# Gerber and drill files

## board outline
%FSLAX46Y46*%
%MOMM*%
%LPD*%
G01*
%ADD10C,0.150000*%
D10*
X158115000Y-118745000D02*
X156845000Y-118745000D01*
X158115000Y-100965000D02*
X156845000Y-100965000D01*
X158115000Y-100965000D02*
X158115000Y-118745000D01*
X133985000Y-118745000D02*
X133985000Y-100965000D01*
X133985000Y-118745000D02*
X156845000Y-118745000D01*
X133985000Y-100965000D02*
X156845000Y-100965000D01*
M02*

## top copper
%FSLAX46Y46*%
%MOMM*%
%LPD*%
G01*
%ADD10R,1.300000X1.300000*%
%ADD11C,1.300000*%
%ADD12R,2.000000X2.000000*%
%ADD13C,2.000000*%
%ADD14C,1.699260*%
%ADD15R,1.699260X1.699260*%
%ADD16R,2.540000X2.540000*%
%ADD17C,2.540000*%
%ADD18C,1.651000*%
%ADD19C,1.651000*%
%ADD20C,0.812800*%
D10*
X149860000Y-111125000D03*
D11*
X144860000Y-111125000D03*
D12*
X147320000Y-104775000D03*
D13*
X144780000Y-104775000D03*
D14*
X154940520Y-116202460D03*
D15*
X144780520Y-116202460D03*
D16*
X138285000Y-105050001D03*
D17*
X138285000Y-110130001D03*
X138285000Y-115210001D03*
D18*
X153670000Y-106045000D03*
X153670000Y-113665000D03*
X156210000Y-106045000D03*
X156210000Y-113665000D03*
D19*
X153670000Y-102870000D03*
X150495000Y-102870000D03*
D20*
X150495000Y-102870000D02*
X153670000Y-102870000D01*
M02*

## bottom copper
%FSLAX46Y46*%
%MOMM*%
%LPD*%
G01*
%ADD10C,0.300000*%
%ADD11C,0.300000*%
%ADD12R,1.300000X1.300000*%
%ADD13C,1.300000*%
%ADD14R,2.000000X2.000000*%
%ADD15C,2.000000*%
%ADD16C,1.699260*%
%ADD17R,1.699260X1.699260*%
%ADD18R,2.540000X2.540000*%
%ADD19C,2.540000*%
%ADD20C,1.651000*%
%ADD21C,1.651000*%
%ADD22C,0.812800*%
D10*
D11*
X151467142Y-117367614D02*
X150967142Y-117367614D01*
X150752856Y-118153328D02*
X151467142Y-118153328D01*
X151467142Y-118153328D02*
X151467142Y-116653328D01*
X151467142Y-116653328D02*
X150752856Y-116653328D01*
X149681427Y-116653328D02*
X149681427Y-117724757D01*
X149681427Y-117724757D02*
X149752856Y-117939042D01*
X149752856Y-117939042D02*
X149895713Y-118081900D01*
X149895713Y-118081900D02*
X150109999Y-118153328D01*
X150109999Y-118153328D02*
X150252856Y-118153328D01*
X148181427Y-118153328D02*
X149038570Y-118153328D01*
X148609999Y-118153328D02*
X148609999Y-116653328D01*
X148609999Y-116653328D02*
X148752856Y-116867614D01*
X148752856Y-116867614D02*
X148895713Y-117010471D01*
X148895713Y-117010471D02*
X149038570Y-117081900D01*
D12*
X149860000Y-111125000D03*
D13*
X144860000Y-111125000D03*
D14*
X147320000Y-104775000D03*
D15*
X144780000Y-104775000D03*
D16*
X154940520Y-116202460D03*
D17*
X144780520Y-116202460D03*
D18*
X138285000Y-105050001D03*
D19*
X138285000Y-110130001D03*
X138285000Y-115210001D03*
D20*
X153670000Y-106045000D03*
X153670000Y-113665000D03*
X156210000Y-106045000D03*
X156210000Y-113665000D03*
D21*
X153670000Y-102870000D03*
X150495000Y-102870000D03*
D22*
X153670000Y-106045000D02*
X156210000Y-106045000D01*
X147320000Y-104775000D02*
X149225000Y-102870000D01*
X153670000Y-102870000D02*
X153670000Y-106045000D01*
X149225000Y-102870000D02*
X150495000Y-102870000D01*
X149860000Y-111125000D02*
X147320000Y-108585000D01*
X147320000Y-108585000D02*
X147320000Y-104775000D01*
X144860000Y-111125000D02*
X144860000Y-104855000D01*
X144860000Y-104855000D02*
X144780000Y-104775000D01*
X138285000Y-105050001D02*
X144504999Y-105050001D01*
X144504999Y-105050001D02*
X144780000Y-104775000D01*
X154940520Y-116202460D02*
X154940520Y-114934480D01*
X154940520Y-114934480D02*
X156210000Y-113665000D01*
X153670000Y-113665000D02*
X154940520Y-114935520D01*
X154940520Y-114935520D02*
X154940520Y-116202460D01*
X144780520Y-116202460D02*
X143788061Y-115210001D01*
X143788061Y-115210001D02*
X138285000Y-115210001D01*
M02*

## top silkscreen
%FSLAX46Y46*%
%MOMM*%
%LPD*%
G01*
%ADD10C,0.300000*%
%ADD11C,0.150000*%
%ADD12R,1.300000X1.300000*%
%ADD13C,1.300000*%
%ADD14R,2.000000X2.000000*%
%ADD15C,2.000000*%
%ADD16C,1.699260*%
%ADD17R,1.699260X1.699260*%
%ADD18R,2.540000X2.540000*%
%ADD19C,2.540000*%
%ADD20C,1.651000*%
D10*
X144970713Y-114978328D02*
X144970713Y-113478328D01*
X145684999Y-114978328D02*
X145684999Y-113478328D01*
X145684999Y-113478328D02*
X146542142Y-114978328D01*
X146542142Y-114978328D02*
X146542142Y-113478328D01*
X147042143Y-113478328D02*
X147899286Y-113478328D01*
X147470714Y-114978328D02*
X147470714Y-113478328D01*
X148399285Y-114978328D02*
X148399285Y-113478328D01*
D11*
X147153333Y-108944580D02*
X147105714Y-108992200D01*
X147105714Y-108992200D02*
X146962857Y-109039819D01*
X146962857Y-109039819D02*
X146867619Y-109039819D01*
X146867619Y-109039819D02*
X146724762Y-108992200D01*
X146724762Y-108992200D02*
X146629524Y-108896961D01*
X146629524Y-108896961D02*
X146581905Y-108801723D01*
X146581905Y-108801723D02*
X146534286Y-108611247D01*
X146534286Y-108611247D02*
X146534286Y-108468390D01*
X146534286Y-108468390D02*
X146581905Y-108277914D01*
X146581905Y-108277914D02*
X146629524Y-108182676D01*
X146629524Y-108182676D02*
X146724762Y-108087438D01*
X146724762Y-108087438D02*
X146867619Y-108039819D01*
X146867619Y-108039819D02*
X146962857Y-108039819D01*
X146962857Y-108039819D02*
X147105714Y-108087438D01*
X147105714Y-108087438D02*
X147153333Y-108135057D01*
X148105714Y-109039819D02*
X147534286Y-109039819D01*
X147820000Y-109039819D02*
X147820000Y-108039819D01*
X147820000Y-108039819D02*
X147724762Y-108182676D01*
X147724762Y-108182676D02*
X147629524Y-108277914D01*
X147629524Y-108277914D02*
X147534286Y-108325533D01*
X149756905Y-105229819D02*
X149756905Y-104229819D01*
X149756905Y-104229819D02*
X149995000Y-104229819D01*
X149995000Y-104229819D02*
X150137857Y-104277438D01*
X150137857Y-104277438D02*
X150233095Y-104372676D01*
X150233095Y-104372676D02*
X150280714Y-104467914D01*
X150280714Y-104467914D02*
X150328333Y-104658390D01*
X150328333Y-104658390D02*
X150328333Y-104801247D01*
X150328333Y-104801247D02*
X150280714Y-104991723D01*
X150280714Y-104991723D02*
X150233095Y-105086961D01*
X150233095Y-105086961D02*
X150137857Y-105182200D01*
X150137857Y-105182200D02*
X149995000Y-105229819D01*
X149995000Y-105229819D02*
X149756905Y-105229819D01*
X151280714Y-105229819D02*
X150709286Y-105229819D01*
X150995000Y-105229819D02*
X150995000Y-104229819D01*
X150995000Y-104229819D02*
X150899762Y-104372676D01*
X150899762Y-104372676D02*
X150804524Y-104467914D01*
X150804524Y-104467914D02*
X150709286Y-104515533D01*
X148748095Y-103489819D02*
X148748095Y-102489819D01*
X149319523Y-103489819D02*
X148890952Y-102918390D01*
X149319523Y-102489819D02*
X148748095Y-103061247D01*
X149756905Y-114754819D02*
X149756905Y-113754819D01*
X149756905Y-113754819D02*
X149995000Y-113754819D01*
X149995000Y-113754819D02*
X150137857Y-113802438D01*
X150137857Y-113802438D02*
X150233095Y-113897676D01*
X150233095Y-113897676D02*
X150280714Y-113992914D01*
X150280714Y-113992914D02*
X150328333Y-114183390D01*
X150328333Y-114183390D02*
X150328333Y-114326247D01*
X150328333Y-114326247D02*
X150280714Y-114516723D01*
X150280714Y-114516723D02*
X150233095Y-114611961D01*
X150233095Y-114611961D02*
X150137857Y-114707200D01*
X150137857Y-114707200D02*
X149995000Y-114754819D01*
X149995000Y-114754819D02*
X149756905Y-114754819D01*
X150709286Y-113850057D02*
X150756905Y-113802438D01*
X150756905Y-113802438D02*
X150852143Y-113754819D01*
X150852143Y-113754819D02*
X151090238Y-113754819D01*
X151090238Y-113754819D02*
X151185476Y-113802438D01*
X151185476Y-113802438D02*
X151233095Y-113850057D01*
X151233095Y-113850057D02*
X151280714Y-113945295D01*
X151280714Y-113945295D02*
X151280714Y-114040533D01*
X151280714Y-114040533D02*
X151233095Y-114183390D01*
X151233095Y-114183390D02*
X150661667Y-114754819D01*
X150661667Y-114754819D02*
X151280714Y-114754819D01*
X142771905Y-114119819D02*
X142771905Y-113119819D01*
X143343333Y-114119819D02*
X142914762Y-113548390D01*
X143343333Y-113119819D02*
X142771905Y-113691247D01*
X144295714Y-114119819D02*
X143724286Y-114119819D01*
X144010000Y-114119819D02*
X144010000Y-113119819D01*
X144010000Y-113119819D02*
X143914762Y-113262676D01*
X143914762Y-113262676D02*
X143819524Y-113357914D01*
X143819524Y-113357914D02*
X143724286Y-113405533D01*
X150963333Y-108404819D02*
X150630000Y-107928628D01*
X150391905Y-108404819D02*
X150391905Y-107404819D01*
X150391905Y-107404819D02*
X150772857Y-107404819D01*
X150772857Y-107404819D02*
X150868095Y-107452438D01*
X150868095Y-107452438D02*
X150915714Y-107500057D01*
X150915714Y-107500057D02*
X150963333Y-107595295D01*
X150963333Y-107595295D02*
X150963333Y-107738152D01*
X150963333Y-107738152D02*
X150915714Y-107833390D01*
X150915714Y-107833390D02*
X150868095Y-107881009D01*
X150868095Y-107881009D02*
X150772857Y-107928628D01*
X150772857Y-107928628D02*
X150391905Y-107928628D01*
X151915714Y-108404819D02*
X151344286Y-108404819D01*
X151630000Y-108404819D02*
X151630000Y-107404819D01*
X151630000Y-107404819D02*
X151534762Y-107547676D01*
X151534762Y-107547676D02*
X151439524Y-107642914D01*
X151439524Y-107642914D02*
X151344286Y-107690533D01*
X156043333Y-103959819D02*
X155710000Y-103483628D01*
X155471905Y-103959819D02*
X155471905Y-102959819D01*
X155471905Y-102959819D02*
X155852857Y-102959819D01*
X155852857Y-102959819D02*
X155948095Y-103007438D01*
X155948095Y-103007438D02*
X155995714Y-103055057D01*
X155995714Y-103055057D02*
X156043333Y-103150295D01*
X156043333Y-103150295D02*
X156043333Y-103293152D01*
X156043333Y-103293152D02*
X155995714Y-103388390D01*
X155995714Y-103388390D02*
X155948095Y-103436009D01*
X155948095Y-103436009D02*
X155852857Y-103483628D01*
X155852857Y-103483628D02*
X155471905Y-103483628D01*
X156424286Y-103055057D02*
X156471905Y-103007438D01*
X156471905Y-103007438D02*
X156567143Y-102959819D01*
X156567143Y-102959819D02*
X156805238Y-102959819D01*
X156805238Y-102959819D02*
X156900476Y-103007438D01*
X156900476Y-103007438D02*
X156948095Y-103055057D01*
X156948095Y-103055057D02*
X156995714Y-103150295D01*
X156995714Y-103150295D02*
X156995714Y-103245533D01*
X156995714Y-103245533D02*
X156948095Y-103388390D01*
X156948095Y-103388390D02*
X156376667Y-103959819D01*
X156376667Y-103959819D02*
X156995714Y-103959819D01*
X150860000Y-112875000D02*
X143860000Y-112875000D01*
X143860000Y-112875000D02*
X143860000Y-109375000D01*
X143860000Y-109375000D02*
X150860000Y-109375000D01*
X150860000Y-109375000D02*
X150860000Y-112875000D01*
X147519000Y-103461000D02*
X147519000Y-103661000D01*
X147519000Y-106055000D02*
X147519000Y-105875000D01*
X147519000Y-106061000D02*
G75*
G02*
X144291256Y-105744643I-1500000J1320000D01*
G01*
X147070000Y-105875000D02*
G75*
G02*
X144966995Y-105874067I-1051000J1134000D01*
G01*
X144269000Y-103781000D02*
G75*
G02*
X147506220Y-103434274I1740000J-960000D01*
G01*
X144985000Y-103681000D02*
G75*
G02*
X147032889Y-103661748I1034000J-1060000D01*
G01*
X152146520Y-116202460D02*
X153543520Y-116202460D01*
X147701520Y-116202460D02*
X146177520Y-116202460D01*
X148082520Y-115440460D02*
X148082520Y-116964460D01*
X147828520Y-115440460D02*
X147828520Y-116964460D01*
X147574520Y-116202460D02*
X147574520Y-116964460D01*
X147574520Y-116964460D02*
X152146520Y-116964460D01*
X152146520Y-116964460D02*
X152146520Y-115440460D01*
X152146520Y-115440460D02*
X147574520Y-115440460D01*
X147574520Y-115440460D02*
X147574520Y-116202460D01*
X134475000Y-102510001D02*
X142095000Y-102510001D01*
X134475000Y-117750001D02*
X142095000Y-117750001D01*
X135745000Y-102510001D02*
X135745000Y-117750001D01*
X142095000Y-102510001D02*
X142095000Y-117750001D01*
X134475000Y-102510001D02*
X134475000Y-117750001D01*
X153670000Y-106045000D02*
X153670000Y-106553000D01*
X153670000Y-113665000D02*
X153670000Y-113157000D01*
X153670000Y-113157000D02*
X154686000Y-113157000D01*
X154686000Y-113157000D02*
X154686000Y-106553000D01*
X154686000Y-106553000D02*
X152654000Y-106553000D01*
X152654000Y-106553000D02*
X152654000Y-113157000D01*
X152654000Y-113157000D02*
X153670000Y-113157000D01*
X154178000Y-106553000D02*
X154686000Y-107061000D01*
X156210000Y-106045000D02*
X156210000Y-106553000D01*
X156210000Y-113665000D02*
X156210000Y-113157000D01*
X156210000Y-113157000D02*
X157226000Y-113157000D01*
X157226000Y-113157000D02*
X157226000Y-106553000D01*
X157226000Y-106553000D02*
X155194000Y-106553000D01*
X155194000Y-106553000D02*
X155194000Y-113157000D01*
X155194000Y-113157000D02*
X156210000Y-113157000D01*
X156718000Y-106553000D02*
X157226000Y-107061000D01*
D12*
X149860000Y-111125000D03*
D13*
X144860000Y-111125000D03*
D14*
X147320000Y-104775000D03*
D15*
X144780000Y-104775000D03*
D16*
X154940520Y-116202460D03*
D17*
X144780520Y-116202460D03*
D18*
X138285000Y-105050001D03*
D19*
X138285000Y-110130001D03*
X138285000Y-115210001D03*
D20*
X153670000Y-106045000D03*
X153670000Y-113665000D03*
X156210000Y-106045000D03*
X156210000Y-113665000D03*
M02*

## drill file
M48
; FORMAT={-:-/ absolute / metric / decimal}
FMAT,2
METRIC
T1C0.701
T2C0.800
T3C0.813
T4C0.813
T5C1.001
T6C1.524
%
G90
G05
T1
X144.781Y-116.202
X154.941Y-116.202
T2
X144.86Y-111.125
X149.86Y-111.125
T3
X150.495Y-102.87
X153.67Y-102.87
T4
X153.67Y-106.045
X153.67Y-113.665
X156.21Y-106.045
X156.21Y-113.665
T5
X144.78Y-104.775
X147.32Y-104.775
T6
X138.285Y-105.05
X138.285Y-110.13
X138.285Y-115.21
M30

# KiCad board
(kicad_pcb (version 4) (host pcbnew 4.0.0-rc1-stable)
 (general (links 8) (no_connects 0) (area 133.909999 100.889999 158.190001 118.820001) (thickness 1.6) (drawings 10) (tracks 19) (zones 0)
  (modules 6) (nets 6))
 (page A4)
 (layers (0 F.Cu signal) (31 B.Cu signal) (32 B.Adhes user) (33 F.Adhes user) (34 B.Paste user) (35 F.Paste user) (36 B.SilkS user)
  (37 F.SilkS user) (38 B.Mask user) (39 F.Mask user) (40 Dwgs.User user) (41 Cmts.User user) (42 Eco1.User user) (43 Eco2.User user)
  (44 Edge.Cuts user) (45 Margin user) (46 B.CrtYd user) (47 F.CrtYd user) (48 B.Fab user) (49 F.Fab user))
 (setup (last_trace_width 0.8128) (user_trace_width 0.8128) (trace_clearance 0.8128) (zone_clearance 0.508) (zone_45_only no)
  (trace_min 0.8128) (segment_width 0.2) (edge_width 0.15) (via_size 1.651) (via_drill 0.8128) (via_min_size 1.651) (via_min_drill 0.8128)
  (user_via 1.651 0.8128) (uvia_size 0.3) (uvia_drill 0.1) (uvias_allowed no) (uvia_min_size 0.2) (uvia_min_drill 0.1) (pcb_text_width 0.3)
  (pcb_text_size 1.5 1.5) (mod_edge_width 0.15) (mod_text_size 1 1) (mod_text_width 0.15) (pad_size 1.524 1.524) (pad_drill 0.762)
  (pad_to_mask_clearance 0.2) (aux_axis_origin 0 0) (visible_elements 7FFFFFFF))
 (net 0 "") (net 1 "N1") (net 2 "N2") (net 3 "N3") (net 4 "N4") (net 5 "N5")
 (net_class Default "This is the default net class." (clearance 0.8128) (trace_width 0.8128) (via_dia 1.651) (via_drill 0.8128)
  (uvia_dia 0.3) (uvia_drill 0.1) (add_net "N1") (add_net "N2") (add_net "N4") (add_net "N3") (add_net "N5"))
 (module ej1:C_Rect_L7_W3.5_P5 (layer F.Cu) (at 149.86 111.125 180)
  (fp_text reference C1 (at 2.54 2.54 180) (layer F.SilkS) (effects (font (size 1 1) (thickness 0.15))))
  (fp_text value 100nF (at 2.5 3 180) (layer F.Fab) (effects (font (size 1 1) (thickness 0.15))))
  (fp_line (start -1 -1.75) (end 6 -1.75) (layer F.SilkS) (width 0.15))
  (fp_line (start 6 -1.75) (end 6 1.75) (layer F.SilkS) (width 0.15))
  (fp_line (start 6 1.75) (end -1 1.75) (layer F.SilkS) (width 0.15))
  (fp_line (start -1 1.75) (end -1 -1.75) (layer F.SilkS) (width 0.15))
  (pad 1 thru_hole rect (at 0 0 180) (size 1.3 1.3) (drill 0.8) (layers *.Cu *.Mask F.SilkS) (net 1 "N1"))
  (pad 2 thru_hole circle (at 5 0 180) (size 1.3 1.3) (drill 0.8) (layers *.Cu *.Mask F.SilkS) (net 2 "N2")))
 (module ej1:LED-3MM (layer F.Cu) (at 147.32 104.775 180)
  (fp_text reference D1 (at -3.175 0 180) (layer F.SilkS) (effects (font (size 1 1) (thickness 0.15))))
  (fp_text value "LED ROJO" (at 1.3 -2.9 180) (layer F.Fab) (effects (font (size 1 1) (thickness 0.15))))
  (fp_line (start -0.199 1.314) (end -0.199 1.114) (layer F.SilkS) (width 0.15))
  (fp_line (start -0.199 -1.28) (end -0.199 -1.1) (layer F.SilkS) (width 0.15))
  (fp_arc (start 1.301 0.034) (end -0.199 -1.286) (angle 108.5) (layer F.SilkS) (width 0.15))
  (fp_arc (start 1.301 0.034) (end 0.25 -1.1) (angle 85.7) (layer F.SilkS) (width 0.15))
  (fp_arc (start 1.311 0.034) (end 3.051 0.994) (angle 110) (layer F.SilkS) (width 0.15))
  (fp_arc (start 1.301 0.034) (end 2.335 1.094) (angle 87.5) (layer F.SilkS) (width 0.15))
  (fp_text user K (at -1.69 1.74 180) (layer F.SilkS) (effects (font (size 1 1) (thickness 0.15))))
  (pad 1 thru_hole rect (at 0 0 270) (size 2 2) (drill 1.00076) (layers *.Cu *.Mask F.SilkS) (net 1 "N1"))
  (pad 2 thru_hole circle (at 2.54 0 180) (size 2 2) (drill 1.00076) (layers *.Cu *.Mask F.SilkS) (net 2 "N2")))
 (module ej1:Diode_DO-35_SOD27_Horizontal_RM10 (layer F.Cu) (at 144.78 116.205)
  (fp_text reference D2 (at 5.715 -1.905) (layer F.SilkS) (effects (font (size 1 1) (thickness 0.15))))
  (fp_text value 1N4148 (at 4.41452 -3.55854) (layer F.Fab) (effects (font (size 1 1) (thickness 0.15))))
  (fp_line (start 7.36652 -0.00254) (end 8.76352 -0.00254) (layer F.SilkS) (width 0.15))
  (fp_line (start 2.92152 -0.00254) (end 1.39752 -0.00254) (layer F.SilkS) (width 0.15))
  (fp_line (start 3.30252 -0.76454) (end 3.30252 0.75946) (layer F.SilkS) (width 0.15))
  (fp_line (start 3.04852 -0.76454) (end 3.04852 0.75946) (layer F.SilkS) (width 0.15))
  (fp_line (start 2.79452 -0.00254) (end 2.79452 0.75946) (layer F.SilkS) (width 0.15))
  (fp_line (start 2.79452 0.75946) (end 7.36652 0.75946) (layer F.SilkS) (width 0.15))
  (fp_line (start 7.36652 0.75946) (end 7.36652 -0.76454) (layer F.SilkS) (width 0.15))
  (fp_line (start 7.36652 -0.76454) (end 2.79452 -0.76454) (layer F.SilkS) (width 0.15))
  (fp_line (start 2.79452 -0.76454) (end 2.79452 -0.00254) (layer F.SilkS) (width 0.15))
  (pad 2 thru_hole circle (at 10.16052 -0.00254 180) (size 1.69926 1.69926) (drill 0.70104) (layers *.Cu *.Mask F.SilkS) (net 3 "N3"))
  (pad 1 thru_hole rect (at 0.00052 -0.00254 180) (size 1.69926 1.69926) (drill 0.70104) (layers *.Cu *.Mask F.SilkS) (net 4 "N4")))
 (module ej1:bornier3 (layer F.Cu) (at 138.285 110.130001 270)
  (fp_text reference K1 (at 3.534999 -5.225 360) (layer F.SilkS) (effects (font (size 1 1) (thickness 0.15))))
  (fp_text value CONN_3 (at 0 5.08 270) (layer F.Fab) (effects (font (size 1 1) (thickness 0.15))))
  (fp_line (start -7.62 3.81) (end -7.62 -3.81) (layer F.SilkS) (width 0.15))
  (fp_line (start 7.62 3.81) (end 7.62 -3.81) (layer F.SilkS) (width 0.15))
  (fp_line (start -7.62 2.54) (end 7.62 2.54) (layer F.SilkS) (width 0.15))
  (fp_line (start -7.62 -3.81) (end 7.62 -3.81) (layer F.SilkS) (width 0.15))
  (fp_line (start -7.62 3.81) (end 7.62 3.81) (layer F.SilkS) (width 0.15))
  (pad 1 thru_hole rect (at -5.08 0 270) (size 2.54 2.54) (drill 1.524) (layers *.Cu *.Mask F.SilkS) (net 2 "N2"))
  (pad 2 thru_hole circle (at 0 0 270) (size 2.54 2.54) (drill 1.524) (layers *.Cu *.Mask F.SilkS) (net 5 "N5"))
  (pad 3 thru_hole circle (at 5.08 0 270) (size 2.54 2.54) (drill 1.524) (layers *.Cu *.Mask F.SilkS) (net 4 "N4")))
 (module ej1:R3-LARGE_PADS (layer F.Cu) (at 153.67 109.855 270)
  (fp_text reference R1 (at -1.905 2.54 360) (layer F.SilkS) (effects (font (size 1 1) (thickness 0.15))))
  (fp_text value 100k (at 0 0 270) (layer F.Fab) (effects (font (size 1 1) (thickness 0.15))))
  (fp_line (start -3.81 0) (end -3.302 0) (layer F.SilkS) (width 0.15))
  (fp_line (start 3.81 0) (end 3.302 0) (layer F.SilkS) (width 0.15))
  (fp_line (start 3.302 0) (end 3.302 -1.016) (layer F.SilkS) (width 0.15))
  (fp_line (start 3.302 -1.016) (end -3.302 -1.016) (layer F.SilkS) (width 0.15))
  (fp_line (start -3.302 -1.016) (end -3.302 1.016) (layer F.SilkS) (width 0.15))
  (fp_line (start -3.302 1.016) (end 3.302 1.016) (layer F.SilkS) (width 0.15))
  (fp_line (start 3.302 1.016) (end 3.302 0) (layer F.SilkS) (width 0.15))
  (fp_line (start -3.302 -0.508) (end -2.794 -1.016) (layer F.SilkS) (width 0.15))
  (pad 1 thru_hole circle (at -3.81 0 270) (size 1.651 1.651) (drill 0.8128) (layers *.Cu *.Mask F.SilkS) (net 1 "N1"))
  (pad 2 thru_hole circle (at 3.81 0 270) (size 1.651 1.651) (drill 0.8128) (layers *.Cu *.Mask F.SilkS) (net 3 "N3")))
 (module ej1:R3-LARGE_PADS (layer F.Cu) (at 156.21 109.855 270)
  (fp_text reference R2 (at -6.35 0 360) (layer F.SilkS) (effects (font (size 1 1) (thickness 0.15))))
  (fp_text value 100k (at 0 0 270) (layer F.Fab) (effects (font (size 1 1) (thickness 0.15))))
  (fp_line (start -3.81 0) (end -3.302 0) (layer F.SilkS) (width 0.15))
  (fp_line (start 3.81 0) (end 3.302 0) (layer F.SilkS) (width 0.15))
  (fp_line (start 3.302 0) (end 3.302 -1.016) (layer F.SilkS) (width 0.15))
  (fp_line (start 3.302 -1.016) (end -3.302 -1.016) (layer F.SilkS) (width 0.15))
  (fp_line (start -3.302 -1.016) (end -3.302 1.016) (layer F.SilkS) (width 0.15))
  (fp_line (start -3.302 1.016) (end 3.302 1.016) (layer F.SilkS) (width 0.15))
  (fp_line (start 3.302 1.016) (end 3.302 0) (layer F.SilkS) (width 0.15))
  (fp_line (start -3.302 -0.508) (end -2.794 -1.016) (layer F.SilkS) (width 0.15))
  (pad 1 thru_hole circle (at -3.81 0 270) (size 1.651 1.651) (drill 0.8128) (layers *.Cu *.Mask F.SilkS) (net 1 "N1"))
  (pad 2 thru_hole circle (at 3.81 0 270) (size 1.651 1.651) (drill 0.8128) (layers *.Cu *.Mask F.SilkS) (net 3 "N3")))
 (gr_line (start 158.115 118.745) (end 156.845 118.745) (angle 90) (layer Edge.Cuts) (width 0.15))
 (gr_line (start 158.115 100.965) (end 156.845 100.965) (angle 90) (layer Edge.Cuts) (width 0.15))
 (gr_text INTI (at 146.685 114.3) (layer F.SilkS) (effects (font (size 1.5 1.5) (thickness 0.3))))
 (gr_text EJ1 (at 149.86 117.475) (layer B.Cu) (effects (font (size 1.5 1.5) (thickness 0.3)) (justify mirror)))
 (gr_line (start 158.115 100.965) (end 158.115 118.745) (angle 90) (layer Edge.Cuts) (width 0.15))
 (gr_line (start 133.985 118.745) (end 133.985 100.965) (angle 90) (layer Edge.Cuts) (width 0.15))
 (gr_line (start 133.985 118.745) (end 156.845 118.745) (angle 90) (layer Edge.Cuts) (width 0.15))
 (gr_line (start 133.985 100.965) (end 156.845 100.965) (angle 90) (layer Edge.Cuts) (width 0.15))
 (segment (start 153.67 106.045) (end 156.21 106.045) (width 0.8128) (layer B.Cu) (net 1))
 (segment (start 147.32 104.775) (end 149.225 102.87) (width 0.8128) (layer B.Cu) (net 1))
 (segment (start 153.67 102.87) (end 153.67 106.045) (width 0.8128) (layer B.Cu) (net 1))
 (via (at 153.67 102.87) (size 1.651) (drill 0.8128) (layers F.Cu B.Cu) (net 1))
 (segment (start 150.495 102.87) (end 153.67 102.87) (width 0.8128) (layer F.Cu) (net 1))
 (via (at 150.495 102.87) (size 1.651) (drill 0.8128) (layers F.Cu B.Cu) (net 1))
 (segment (start 149.225 102.87) (end 150.495 102.87) (width 0.8128) (layer B.Cu) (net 1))
 (segment (start 149.86 111.125) (end 147.32 108.585) (width 0.8128) (layer B.Cu) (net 1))
 (segment (start 147.32 108.585) (end 147.32 104.775) (width 0.8128) (layer B.Cu) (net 1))
 (segment (start 144.86 111.125) (end 144.86 104.855) (width 0.8128) (layer B.Cu) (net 2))
 (segment (start 144.86 104.855) (end 144.78 104.775) (width 0.8128) (layer B.Cu) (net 2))
 (segment (start 138.285 105.050001) (end 144.504999 105.050001) (width 0.8128) (layer B.Cu) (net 2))
 (segment (start 144.504999 105.050001) (end 144.78 104.775) (width 0.8128) (layer B.Cu) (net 2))
 (segment (start 154.94052 116.20246) (end 154.94052 114.93448) (width 0.8128) (layer B.Cu) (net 3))
 (segment (start 154.94052 114.93448) (end 156.21 113.665) (width 0.8128) (layer B.Cu) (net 3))
 (segment (start 153.67 113.665) (end 154.94052 114.93552) (width 0.8128) (layer B.Cu) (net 3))
 (segment (start 154.94052 114.93552) (end 154.94052 116.20246) (width 0.8128) (layer B.Cu) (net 3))
 (segment (start 144.78052 116.20246) (end 143.788061 115.210001) (width 0.8128) (layer B.Cu) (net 4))
 (segment (start 143.788061 115.210001) (end 138.285 115.210001) (width 0.8128) (layer B.Cu) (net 4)))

